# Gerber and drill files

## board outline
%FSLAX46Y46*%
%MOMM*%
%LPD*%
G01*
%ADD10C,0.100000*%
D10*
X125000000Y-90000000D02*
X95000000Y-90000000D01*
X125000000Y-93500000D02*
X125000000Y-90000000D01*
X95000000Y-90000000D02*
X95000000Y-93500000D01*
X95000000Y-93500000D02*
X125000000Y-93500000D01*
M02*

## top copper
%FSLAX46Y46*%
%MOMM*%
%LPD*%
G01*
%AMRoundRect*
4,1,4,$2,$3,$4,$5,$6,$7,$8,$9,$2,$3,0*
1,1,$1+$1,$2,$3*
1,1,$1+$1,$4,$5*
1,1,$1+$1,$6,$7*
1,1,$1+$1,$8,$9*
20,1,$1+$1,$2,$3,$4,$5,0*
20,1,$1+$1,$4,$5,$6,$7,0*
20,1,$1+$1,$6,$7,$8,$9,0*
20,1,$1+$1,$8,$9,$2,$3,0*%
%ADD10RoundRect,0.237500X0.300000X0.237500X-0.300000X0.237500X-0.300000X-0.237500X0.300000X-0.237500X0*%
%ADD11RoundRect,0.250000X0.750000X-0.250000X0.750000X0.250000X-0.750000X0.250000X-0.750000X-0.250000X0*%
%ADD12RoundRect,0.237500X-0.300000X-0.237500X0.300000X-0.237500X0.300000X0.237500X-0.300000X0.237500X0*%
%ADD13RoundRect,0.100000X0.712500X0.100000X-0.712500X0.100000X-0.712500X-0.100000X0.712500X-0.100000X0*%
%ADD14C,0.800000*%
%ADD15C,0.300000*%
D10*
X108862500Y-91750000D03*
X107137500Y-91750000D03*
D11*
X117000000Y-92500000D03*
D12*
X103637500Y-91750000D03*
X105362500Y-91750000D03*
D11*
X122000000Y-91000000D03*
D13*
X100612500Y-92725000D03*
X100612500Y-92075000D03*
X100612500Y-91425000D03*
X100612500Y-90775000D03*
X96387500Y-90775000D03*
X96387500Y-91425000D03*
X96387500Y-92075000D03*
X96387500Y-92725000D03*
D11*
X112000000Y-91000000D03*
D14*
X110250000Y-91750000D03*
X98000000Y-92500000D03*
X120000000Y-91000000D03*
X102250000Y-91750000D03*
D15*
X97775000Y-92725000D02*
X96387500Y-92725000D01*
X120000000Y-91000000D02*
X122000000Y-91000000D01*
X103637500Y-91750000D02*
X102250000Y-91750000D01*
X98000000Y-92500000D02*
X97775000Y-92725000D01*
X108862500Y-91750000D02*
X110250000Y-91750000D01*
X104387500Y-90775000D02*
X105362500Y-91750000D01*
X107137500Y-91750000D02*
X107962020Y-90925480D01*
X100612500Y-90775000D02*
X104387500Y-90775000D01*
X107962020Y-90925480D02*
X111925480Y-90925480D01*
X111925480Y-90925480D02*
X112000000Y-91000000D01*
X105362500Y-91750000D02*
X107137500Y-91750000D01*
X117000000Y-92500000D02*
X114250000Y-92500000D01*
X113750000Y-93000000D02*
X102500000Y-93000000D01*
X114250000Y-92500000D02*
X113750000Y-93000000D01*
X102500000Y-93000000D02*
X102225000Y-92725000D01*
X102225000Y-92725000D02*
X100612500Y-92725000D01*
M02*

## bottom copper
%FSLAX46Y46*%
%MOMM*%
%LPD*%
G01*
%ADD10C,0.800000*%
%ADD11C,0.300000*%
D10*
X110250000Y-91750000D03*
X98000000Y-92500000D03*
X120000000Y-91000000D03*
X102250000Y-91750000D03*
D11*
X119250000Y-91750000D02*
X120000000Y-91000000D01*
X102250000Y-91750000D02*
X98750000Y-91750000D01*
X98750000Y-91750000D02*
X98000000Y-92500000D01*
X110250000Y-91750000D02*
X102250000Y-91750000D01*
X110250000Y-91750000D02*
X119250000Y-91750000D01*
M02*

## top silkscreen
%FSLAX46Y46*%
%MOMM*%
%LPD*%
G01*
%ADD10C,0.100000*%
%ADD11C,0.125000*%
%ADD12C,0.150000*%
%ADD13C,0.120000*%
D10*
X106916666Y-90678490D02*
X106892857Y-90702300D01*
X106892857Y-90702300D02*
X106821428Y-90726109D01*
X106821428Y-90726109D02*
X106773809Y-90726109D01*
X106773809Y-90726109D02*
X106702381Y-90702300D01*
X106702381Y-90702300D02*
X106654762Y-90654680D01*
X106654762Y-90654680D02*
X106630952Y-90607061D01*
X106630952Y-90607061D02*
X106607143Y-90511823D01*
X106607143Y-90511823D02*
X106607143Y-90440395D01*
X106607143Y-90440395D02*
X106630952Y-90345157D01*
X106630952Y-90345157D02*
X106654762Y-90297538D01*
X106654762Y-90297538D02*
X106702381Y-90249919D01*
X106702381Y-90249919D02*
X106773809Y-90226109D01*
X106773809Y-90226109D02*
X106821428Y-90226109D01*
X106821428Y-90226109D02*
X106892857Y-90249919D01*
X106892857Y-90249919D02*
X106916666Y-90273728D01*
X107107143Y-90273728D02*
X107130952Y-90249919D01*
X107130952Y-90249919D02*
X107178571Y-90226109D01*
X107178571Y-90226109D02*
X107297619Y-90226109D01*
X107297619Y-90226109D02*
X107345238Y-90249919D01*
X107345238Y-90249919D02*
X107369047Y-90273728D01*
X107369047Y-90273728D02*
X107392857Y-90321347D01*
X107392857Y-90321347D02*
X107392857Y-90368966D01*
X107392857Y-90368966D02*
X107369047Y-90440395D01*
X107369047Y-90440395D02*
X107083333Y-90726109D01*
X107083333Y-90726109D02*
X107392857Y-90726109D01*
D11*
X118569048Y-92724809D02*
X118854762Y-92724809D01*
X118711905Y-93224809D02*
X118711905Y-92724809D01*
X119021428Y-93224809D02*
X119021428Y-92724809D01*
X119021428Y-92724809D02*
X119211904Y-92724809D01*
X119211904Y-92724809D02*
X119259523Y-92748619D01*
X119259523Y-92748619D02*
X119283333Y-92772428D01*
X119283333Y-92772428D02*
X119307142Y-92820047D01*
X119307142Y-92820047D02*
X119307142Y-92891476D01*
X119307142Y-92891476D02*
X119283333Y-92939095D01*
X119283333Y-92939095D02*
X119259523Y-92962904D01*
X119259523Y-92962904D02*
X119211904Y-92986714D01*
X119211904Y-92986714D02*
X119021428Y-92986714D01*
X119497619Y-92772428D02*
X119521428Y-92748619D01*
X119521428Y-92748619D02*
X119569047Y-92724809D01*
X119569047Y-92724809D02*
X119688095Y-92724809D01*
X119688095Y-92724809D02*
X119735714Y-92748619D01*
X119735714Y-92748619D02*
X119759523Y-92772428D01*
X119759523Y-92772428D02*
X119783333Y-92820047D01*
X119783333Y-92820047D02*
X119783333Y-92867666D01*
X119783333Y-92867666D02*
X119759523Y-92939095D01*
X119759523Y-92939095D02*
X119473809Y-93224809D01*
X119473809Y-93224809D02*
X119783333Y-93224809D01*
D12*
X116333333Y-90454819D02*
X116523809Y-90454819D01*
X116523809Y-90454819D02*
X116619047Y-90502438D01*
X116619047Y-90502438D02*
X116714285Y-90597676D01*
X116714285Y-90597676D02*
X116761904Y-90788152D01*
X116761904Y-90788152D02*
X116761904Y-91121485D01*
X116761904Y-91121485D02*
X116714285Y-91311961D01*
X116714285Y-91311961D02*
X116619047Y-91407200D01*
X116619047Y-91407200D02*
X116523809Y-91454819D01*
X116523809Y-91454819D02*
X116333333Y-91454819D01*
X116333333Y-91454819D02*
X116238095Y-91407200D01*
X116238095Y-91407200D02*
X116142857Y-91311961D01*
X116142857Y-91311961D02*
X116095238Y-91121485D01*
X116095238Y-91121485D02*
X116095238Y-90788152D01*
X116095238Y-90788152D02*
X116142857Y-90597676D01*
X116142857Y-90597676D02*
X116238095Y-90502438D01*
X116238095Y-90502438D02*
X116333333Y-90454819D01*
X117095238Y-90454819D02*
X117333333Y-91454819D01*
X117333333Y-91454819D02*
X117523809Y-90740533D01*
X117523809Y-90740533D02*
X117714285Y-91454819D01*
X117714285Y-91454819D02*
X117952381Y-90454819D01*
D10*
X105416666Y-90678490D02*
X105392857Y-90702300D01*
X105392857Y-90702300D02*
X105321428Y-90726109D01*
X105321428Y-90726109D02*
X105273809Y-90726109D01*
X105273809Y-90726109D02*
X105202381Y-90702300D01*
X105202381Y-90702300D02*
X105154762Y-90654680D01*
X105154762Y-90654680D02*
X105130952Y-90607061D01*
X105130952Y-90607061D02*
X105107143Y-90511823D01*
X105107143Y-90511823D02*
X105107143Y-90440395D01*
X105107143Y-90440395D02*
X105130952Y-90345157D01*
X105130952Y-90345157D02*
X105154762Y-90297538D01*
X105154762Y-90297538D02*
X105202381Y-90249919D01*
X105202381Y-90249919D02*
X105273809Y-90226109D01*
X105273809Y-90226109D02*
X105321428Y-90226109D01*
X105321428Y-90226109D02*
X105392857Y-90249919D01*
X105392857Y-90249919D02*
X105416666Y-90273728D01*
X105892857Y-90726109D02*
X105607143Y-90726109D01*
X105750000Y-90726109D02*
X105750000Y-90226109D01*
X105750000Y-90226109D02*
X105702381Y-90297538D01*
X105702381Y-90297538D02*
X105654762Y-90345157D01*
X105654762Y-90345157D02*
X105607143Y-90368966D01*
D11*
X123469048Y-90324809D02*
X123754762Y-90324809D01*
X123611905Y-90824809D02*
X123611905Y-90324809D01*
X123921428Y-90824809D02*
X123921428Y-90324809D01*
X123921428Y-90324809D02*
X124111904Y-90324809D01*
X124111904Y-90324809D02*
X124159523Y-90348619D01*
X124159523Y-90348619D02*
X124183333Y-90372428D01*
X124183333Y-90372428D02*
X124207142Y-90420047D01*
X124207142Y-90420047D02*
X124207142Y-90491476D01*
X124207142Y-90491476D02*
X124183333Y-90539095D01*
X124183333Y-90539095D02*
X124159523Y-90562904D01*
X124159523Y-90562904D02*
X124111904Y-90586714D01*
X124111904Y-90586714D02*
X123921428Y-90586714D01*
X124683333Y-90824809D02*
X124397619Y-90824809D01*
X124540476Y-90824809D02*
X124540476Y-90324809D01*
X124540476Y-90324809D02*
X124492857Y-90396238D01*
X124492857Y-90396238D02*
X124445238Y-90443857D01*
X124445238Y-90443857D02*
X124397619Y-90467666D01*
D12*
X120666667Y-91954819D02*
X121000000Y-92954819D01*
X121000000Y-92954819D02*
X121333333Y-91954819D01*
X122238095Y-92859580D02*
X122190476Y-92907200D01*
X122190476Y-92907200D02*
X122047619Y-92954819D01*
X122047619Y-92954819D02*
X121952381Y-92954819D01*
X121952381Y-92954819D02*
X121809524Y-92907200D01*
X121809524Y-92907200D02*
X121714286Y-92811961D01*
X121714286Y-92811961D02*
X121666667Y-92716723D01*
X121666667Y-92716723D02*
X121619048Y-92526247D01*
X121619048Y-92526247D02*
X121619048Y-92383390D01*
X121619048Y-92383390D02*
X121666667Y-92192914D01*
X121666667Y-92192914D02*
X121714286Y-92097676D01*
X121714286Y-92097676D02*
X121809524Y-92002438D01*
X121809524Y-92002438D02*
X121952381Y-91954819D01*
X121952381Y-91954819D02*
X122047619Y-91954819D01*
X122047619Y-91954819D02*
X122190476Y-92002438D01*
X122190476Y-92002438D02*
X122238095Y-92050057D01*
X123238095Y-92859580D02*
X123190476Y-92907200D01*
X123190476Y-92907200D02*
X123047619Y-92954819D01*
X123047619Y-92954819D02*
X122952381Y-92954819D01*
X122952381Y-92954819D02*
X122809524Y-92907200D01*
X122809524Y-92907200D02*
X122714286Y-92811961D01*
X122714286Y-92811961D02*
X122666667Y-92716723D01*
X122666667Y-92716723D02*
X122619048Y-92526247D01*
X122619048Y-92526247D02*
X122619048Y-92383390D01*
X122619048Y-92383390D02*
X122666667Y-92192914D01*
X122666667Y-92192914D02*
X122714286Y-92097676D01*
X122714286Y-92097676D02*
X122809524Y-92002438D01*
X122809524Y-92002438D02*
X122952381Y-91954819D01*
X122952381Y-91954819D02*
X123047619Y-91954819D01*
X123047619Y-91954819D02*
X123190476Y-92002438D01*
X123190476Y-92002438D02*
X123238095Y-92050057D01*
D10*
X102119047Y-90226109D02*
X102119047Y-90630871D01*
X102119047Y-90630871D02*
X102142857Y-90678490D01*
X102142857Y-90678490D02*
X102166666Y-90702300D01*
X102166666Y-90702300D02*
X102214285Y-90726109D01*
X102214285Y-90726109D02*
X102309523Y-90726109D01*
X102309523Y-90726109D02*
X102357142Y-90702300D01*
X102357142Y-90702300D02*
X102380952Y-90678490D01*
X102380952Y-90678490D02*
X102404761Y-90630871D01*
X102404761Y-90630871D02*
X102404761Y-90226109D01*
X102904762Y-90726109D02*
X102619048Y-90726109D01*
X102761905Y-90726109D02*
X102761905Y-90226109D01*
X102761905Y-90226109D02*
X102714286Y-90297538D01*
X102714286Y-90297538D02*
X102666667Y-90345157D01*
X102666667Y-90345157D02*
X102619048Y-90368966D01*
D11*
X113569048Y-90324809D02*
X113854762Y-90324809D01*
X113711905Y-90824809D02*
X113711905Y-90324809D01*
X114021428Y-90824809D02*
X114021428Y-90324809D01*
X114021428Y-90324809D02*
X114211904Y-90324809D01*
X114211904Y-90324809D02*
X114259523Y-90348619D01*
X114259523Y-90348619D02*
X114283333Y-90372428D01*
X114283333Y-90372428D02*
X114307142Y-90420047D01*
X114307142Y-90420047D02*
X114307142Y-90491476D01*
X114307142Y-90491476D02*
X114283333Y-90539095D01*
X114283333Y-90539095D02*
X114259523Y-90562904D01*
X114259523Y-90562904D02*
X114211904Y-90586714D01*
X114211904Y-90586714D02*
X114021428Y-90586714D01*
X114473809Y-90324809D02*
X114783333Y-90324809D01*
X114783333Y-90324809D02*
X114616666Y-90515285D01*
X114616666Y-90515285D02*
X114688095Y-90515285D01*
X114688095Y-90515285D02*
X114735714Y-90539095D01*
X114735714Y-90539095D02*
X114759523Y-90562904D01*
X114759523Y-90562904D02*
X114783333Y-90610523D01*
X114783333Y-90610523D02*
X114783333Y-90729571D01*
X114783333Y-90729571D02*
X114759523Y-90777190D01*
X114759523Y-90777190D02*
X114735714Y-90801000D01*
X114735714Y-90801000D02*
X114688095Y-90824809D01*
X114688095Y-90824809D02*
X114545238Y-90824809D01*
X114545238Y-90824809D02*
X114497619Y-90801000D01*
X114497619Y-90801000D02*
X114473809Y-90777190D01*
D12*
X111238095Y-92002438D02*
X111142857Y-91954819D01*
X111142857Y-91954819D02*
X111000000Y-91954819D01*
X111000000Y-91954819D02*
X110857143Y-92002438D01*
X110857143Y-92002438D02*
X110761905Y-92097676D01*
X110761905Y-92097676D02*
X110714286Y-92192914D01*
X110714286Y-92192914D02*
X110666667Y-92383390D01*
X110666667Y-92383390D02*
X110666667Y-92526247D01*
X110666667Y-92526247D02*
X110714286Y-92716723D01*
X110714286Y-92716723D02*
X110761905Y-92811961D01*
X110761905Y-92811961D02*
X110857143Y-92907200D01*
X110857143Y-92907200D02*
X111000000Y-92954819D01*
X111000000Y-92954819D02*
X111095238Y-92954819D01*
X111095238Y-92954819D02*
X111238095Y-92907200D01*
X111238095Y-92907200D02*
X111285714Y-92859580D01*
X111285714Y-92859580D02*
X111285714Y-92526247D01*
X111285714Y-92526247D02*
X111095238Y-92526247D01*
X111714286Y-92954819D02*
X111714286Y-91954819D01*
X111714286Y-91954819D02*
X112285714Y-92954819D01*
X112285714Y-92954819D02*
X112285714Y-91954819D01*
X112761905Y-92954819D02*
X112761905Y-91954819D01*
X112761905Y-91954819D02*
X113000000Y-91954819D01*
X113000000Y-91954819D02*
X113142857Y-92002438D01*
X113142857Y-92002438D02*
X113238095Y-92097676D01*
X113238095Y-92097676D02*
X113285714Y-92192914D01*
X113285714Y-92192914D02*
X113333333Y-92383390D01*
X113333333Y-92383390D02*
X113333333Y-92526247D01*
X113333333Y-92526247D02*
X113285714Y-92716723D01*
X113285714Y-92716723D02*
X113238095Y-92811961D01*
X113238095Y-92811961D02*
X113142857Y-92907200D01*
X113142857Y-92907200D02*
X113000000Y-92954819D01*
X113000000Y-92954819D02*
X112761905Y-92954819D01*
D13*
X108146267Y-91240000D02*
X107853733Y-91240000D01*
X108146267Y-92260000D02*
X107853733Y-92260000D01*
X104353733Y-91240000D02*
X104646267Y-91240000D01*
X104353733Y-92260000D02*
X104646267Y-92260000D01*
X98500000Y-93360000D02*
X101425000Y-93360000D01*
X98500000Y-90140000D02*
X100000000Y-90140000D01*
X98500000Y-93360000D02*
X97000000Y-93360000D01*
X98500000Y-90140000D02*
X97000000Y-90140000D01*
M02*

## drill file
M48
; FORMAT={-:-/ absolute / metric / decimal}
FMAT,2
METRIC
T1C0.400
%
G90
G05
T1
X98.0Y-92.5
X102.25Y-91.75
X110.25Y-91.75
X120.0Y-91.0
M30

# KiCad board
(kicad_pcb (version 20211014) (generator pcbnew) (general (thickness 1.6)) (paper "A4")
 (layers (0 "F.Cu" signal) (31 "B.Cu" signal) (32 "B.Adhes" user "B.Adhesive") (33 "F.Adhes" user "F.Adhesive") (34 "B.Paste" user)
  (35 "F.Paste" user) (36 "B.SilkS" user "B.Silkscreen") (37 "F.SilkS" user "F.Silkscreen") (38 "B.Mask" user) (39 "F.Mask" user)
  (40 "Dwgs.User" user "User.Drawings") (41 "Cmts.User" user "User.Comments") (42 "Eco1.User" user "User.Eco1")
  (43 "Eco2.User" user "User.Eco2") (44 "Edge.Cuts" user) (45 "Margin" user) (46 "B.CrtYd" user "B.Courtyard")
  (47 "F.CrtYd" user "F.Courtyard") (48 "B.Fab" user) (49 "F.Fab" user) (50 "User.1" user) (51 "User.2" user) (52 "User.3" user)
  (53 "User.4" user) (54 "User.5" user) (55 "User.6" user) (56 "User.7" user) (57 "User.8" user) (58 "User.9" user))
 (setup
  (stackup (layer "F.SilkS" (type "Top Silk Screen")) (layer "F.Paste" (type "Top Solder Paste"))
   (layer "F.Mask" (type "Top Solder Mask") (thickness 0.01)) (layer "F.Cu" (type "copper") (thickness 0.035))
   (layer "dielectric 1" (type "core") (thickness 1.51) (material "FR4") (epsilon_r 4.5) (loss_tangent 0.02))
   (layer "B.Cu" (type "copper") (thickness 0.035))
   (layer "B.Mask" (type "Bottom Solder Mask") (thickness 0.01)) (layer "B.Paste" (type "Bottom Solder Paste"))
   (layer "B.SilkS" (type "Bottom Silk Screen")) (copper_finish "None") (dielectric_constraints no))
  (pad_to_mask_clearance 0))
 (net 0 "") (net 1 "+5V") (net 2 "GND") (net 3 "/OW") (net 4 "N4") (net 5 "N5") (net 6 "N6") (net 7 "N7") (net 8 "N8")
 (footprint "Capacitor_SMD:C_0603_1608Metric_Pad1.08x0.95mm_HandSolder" (layer "F.Cu") (at 108 91.75 180)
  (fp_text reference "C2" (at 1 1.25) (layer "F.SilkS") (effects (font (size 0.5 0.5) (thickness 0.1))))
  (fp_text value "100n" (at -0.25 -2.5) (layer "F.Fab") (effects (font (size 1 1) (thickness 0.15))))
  (fp_line (start -0.146267 0.51) (end 0.146267 0.51) (layer "F.SilkS") (width 0.12))
  (fp_line (start -0.146267 -0.51) (end 0.146267 -0.51) (layer "F.SilkS") (width 0.12))
  (pad "1" smd roundrect (at -0.8625 0 180) (size 1.075 0.95) (layers "F.Cu" "F.Paste" "F.Mask") (roundrect_rratio 0.25) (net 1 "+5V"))
  (pad "2" smd roundrect (at 0.8625 0 180) (size 1.075 0.95) (layers "F.Cu" "F.Paste" "F.Mask") (roundrect_rratio 0.25) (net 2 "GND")))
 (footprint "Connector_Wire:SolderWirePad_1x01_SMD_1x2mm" (layer "F.Cu") (at 117 92.5 90)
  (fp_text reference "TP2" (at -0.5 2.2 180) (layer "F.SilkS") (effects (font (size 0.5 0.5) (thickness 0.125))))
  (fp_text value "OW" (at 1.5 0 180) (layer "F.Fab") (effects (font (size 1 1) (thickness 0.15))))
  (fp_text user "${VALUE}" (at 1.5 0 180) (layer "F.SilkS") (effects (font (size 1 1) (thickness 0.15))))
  (pad "1" smd roundrect (at 0 0 90) (size 1 2) (layers "F.Cu" "F.Paste" "F.Mask") (roundrect_rratio 0.25) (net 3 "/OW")))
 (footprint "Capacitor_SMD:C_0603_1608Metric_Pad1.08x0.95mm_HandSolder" (layer "F.Cu") (at 104.5 91.75)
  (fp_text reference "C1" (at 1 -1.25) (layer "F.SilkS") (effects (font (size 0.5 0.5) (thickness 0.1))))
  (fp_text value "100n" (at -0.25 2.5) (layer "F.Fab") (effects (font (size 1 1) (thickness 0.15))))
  (fp_line (start -0.146267 -0.51) (end 0.146267 -0.51) (layer "F.SilkS") (width 0.12))
  (fp_line (start -0.146267 0.51) (end 0.146267 0.51) (layer "F.SilkS") (width 0.12))
  (pad "1" smd roundrect (at -0.8625 0) (size 1.075 0.95) (layers "F.Cu" "F.Paste" "F.Mask") (roundrect_rratio 0.25) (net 1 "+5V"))
  (pad "2" smd roundrect (at 0.8625 0) (size 1.075 0.95) (layers "F.Cu" "F.Paste" "F.Mask") (roundrect_rratio 0.25) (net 2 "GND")))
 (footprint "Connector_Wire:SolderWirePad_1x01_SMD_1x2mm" (layer "F.Cu") (at 122 91 90)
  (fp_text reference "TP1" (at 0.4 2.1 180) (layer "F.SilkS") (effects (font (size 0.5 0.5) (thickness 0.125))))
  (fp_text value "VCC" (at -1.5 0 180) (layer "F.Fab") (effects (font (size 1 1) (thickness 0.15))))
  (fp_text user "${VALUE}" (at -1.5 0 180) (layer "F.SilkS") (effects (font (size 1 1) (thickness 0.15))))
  (pad "1" smd roundrect (at 0 0 90) (size 1 2) (layers "F.Cu" "F.Paste" "F.Mask") (roundrect_rratio 0.25) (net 1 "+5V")))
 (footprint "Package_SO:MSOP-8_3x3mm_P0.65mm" (layer "F.Cu") (at 98.5 91.75 180)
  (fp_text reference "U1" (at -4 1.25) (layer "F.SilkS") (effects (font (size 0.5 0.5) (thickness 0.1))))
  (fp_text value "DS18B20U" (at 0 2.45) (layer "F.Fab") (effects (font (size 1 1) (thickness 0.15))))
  (fp_line (start 0 -1.61) (end -2.925 -1.61) (layer "F.SilkS") (width 0.12))
  (fp_line (start 0 1.61) (end -1.5 1.61) (layer "F.SilkS") (width 0.12))
  (fp_line (start 0 -1.61) (end 1.5 -1.61) (layer "F.SilkS") (width 0.12))
  (fp_line (start 0 1.61) (end 1.5 1.61) (layer "F.SilkS") (width 0.12))
  (pad "1" smd roundrect (at -2.1125 -0.975 180) (size 1.625 0.4) (layers "F.Cu" "F.Paste" "F.Mask") (roundrect_rratio 0.25) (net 3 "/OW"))
  (pad "2" smd roundrect (at -2.1125 -0.325 180) (size 1.625 0.4) (layers "F.Cu" "F.Paste" "F.Mask") (roundrect_rratio 0.25) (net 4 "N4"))
  (pad "3" smd roundrect (at -2.1125 0.325 180) (size 1.625 0.4) (layers "F.Cu" "F.Paste" "F.Mask") (roundrect_rratio 0.25) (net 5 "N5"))
  (pad "4" smd roundrect (at -2.1125 0.975 180) (size 1.625 0.4) (layers "F.Cu" "F.Paste" "F.Mask") (roundrect_rratio 0.25) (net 2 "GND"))
  (pad "5" smd roundrect (at 2.1125 0.975 180) (size 1.625 0.4) (layers "F.Cu" "F.Paste" "F.Mask") (roundrect_rratio 0.25) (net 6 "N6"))
  (pad "6" smd roundrect (at 2.1125 0.325 180) (size 1.625 0.4) (layers "F.Cu" "F.Paste" "F.Mask") (roundrect_rratio 0.25) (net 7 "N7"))
  (pad "7" smd roundrect (at 2.1125 -0.325 180) (size 1.625 0.4) (layers "F.Cu" "F.Paste" "F.Mask") (roundrect_rratio 0.25) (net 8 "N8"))
  (pad "8" smd roundrect (at 2.1125 -0.975 180) (size 1.625 0.4) (layers "F.Cu" "F.Paste" "F.Mask") (roundrect_rratio 0.25) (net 1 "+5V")))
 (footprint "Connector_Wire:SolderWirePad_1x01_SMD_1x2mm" (layer "F.Cu") (at 112 91 90)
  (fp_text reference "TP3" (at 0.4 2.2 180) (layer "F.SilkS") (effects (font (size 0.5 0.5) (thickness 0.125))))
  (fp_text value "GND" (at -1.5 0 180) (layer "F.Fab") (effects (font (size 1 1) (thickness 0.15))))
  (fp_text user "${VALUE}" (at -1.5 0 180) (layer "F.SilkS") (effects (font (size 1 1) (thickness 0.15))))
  (pad "1" smd roundrect (at 0 0 90) (size 1 2) (layers "F.Cu" "F.Paste" "F.Mask") (roundrect_rratio 0.25) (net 2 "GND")))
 (gr_line (start 125 90) (end 95 90) (layer "Edge.Cuts") (width 0.1))
 (gr_line (start 125 93.5) (end 125 90) (layer "Edge.Cuts") (width 0.1))
 (gr_line (start 95 90) (end 95 93.5) (layer "Edge.Cuts") (width 0.1))
 (gr_line (start 95 93.5) (end 125 93.5) (layer "Edge.Cuts") (width 0.1))
 (segment (start 97.775 92.725) (end 96.3875 92.725) (width 0.3) (layer "F.Cu") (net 1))
 (segment (start 120 91) (end 122 91) (width 0.3) (layer "F.Cu") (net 1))
 (segment (start 103.6375 91.75) (end 102.25 91.75) (width 0.3) (layer "F.Cu") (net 1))
 (segment (start 98 92.5) (end 97.775 92.725) (width 0.3) (layer "F.Cu") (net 1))
 (segment (start 108.8625 91.75) (end 110.25 91.75) (width 0.3) (layer "F.Cu") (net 1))
 (via (at 110.25 91.75) (size 0.8) (drill 0.4) (layers "F.Cu" "B.Cu") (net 1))
 (via (at 98 92.5) (size 0.8) (drill 0.4) (layers "F.Cu" "B.Cu") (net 1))
 (via (at 120 91) (size 0.8) (drill 0.4) (layers "F.Cu" "B.Cu") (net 1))
 (via (at 102.25 91.75) (size 0.8) (drill 0.4) (layers "F.Cu" "B.Cu") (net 1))
 (segment (start 119.25 91.75) (end 120 91) (width 0.3) (layer "B.Cu") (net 1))
 (segment (start 102.25 91.75) (end 98.75 91.75) (width 0.3) (layer "B.Cu") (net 1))
 (segment (start 98.75 91.75) (end 98 92.5) (width 0.3) (layer "B.Cu") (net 1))
 (segment (start 110.25 91.75) (end 102.25 91.75) (width 0.3) (layer "B.Cu") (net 1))
 (segment (start 110.25 91.75) (end 119.25 91.75) (width 0.3) (layer "B.Cu") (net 1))
 (segment (start 104.3875 90.775) (end 105.3625 91.75) (width 0.3) (layer "F.Cu") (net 2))
 (segment (start 107.1375 91.75) (end 107.96202 90.92548) (width 0.3) (layer "F.Cu") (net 2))
 (segment (start 100.6125 90.775) (end 104.3875 90.775) (width 0.3) (layer "F.Cu") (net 2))
 (segment (start 107.96202 90.92548) (end 111.92548 90.92548) (width 0.3) (layer "F.Cu") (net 2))
 (segment (start 111.92548 90.92548) (end 112 91) (width 0.3) (layer "F.Cu") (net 2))
 (segment (start 105.3625 91.75) (end 107.1375 91.75) (width 0.3) (layer "F.Cu") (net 2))
 (segment (start 117 92.5) (end 114.25 92.5) (width 0.3) (layer "F.Cu") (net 3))
 (segment (start 113.75 93) (end 102.5 93) (width 0.3) (layer "F.Cu") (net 3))
 (segment (start 114.25 92.5) (end 113.75 93) (width 0.3) (layer "F.Cu") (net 3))
 (segment (start 102.5 93) (end 102.225 92.725) (width 0.3) (layer "F.Cu") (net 3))
 (segment (start 102.225 92.725) (end 100.6125 92.725) (width 0.3) (layer "F.Cu") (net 3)))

